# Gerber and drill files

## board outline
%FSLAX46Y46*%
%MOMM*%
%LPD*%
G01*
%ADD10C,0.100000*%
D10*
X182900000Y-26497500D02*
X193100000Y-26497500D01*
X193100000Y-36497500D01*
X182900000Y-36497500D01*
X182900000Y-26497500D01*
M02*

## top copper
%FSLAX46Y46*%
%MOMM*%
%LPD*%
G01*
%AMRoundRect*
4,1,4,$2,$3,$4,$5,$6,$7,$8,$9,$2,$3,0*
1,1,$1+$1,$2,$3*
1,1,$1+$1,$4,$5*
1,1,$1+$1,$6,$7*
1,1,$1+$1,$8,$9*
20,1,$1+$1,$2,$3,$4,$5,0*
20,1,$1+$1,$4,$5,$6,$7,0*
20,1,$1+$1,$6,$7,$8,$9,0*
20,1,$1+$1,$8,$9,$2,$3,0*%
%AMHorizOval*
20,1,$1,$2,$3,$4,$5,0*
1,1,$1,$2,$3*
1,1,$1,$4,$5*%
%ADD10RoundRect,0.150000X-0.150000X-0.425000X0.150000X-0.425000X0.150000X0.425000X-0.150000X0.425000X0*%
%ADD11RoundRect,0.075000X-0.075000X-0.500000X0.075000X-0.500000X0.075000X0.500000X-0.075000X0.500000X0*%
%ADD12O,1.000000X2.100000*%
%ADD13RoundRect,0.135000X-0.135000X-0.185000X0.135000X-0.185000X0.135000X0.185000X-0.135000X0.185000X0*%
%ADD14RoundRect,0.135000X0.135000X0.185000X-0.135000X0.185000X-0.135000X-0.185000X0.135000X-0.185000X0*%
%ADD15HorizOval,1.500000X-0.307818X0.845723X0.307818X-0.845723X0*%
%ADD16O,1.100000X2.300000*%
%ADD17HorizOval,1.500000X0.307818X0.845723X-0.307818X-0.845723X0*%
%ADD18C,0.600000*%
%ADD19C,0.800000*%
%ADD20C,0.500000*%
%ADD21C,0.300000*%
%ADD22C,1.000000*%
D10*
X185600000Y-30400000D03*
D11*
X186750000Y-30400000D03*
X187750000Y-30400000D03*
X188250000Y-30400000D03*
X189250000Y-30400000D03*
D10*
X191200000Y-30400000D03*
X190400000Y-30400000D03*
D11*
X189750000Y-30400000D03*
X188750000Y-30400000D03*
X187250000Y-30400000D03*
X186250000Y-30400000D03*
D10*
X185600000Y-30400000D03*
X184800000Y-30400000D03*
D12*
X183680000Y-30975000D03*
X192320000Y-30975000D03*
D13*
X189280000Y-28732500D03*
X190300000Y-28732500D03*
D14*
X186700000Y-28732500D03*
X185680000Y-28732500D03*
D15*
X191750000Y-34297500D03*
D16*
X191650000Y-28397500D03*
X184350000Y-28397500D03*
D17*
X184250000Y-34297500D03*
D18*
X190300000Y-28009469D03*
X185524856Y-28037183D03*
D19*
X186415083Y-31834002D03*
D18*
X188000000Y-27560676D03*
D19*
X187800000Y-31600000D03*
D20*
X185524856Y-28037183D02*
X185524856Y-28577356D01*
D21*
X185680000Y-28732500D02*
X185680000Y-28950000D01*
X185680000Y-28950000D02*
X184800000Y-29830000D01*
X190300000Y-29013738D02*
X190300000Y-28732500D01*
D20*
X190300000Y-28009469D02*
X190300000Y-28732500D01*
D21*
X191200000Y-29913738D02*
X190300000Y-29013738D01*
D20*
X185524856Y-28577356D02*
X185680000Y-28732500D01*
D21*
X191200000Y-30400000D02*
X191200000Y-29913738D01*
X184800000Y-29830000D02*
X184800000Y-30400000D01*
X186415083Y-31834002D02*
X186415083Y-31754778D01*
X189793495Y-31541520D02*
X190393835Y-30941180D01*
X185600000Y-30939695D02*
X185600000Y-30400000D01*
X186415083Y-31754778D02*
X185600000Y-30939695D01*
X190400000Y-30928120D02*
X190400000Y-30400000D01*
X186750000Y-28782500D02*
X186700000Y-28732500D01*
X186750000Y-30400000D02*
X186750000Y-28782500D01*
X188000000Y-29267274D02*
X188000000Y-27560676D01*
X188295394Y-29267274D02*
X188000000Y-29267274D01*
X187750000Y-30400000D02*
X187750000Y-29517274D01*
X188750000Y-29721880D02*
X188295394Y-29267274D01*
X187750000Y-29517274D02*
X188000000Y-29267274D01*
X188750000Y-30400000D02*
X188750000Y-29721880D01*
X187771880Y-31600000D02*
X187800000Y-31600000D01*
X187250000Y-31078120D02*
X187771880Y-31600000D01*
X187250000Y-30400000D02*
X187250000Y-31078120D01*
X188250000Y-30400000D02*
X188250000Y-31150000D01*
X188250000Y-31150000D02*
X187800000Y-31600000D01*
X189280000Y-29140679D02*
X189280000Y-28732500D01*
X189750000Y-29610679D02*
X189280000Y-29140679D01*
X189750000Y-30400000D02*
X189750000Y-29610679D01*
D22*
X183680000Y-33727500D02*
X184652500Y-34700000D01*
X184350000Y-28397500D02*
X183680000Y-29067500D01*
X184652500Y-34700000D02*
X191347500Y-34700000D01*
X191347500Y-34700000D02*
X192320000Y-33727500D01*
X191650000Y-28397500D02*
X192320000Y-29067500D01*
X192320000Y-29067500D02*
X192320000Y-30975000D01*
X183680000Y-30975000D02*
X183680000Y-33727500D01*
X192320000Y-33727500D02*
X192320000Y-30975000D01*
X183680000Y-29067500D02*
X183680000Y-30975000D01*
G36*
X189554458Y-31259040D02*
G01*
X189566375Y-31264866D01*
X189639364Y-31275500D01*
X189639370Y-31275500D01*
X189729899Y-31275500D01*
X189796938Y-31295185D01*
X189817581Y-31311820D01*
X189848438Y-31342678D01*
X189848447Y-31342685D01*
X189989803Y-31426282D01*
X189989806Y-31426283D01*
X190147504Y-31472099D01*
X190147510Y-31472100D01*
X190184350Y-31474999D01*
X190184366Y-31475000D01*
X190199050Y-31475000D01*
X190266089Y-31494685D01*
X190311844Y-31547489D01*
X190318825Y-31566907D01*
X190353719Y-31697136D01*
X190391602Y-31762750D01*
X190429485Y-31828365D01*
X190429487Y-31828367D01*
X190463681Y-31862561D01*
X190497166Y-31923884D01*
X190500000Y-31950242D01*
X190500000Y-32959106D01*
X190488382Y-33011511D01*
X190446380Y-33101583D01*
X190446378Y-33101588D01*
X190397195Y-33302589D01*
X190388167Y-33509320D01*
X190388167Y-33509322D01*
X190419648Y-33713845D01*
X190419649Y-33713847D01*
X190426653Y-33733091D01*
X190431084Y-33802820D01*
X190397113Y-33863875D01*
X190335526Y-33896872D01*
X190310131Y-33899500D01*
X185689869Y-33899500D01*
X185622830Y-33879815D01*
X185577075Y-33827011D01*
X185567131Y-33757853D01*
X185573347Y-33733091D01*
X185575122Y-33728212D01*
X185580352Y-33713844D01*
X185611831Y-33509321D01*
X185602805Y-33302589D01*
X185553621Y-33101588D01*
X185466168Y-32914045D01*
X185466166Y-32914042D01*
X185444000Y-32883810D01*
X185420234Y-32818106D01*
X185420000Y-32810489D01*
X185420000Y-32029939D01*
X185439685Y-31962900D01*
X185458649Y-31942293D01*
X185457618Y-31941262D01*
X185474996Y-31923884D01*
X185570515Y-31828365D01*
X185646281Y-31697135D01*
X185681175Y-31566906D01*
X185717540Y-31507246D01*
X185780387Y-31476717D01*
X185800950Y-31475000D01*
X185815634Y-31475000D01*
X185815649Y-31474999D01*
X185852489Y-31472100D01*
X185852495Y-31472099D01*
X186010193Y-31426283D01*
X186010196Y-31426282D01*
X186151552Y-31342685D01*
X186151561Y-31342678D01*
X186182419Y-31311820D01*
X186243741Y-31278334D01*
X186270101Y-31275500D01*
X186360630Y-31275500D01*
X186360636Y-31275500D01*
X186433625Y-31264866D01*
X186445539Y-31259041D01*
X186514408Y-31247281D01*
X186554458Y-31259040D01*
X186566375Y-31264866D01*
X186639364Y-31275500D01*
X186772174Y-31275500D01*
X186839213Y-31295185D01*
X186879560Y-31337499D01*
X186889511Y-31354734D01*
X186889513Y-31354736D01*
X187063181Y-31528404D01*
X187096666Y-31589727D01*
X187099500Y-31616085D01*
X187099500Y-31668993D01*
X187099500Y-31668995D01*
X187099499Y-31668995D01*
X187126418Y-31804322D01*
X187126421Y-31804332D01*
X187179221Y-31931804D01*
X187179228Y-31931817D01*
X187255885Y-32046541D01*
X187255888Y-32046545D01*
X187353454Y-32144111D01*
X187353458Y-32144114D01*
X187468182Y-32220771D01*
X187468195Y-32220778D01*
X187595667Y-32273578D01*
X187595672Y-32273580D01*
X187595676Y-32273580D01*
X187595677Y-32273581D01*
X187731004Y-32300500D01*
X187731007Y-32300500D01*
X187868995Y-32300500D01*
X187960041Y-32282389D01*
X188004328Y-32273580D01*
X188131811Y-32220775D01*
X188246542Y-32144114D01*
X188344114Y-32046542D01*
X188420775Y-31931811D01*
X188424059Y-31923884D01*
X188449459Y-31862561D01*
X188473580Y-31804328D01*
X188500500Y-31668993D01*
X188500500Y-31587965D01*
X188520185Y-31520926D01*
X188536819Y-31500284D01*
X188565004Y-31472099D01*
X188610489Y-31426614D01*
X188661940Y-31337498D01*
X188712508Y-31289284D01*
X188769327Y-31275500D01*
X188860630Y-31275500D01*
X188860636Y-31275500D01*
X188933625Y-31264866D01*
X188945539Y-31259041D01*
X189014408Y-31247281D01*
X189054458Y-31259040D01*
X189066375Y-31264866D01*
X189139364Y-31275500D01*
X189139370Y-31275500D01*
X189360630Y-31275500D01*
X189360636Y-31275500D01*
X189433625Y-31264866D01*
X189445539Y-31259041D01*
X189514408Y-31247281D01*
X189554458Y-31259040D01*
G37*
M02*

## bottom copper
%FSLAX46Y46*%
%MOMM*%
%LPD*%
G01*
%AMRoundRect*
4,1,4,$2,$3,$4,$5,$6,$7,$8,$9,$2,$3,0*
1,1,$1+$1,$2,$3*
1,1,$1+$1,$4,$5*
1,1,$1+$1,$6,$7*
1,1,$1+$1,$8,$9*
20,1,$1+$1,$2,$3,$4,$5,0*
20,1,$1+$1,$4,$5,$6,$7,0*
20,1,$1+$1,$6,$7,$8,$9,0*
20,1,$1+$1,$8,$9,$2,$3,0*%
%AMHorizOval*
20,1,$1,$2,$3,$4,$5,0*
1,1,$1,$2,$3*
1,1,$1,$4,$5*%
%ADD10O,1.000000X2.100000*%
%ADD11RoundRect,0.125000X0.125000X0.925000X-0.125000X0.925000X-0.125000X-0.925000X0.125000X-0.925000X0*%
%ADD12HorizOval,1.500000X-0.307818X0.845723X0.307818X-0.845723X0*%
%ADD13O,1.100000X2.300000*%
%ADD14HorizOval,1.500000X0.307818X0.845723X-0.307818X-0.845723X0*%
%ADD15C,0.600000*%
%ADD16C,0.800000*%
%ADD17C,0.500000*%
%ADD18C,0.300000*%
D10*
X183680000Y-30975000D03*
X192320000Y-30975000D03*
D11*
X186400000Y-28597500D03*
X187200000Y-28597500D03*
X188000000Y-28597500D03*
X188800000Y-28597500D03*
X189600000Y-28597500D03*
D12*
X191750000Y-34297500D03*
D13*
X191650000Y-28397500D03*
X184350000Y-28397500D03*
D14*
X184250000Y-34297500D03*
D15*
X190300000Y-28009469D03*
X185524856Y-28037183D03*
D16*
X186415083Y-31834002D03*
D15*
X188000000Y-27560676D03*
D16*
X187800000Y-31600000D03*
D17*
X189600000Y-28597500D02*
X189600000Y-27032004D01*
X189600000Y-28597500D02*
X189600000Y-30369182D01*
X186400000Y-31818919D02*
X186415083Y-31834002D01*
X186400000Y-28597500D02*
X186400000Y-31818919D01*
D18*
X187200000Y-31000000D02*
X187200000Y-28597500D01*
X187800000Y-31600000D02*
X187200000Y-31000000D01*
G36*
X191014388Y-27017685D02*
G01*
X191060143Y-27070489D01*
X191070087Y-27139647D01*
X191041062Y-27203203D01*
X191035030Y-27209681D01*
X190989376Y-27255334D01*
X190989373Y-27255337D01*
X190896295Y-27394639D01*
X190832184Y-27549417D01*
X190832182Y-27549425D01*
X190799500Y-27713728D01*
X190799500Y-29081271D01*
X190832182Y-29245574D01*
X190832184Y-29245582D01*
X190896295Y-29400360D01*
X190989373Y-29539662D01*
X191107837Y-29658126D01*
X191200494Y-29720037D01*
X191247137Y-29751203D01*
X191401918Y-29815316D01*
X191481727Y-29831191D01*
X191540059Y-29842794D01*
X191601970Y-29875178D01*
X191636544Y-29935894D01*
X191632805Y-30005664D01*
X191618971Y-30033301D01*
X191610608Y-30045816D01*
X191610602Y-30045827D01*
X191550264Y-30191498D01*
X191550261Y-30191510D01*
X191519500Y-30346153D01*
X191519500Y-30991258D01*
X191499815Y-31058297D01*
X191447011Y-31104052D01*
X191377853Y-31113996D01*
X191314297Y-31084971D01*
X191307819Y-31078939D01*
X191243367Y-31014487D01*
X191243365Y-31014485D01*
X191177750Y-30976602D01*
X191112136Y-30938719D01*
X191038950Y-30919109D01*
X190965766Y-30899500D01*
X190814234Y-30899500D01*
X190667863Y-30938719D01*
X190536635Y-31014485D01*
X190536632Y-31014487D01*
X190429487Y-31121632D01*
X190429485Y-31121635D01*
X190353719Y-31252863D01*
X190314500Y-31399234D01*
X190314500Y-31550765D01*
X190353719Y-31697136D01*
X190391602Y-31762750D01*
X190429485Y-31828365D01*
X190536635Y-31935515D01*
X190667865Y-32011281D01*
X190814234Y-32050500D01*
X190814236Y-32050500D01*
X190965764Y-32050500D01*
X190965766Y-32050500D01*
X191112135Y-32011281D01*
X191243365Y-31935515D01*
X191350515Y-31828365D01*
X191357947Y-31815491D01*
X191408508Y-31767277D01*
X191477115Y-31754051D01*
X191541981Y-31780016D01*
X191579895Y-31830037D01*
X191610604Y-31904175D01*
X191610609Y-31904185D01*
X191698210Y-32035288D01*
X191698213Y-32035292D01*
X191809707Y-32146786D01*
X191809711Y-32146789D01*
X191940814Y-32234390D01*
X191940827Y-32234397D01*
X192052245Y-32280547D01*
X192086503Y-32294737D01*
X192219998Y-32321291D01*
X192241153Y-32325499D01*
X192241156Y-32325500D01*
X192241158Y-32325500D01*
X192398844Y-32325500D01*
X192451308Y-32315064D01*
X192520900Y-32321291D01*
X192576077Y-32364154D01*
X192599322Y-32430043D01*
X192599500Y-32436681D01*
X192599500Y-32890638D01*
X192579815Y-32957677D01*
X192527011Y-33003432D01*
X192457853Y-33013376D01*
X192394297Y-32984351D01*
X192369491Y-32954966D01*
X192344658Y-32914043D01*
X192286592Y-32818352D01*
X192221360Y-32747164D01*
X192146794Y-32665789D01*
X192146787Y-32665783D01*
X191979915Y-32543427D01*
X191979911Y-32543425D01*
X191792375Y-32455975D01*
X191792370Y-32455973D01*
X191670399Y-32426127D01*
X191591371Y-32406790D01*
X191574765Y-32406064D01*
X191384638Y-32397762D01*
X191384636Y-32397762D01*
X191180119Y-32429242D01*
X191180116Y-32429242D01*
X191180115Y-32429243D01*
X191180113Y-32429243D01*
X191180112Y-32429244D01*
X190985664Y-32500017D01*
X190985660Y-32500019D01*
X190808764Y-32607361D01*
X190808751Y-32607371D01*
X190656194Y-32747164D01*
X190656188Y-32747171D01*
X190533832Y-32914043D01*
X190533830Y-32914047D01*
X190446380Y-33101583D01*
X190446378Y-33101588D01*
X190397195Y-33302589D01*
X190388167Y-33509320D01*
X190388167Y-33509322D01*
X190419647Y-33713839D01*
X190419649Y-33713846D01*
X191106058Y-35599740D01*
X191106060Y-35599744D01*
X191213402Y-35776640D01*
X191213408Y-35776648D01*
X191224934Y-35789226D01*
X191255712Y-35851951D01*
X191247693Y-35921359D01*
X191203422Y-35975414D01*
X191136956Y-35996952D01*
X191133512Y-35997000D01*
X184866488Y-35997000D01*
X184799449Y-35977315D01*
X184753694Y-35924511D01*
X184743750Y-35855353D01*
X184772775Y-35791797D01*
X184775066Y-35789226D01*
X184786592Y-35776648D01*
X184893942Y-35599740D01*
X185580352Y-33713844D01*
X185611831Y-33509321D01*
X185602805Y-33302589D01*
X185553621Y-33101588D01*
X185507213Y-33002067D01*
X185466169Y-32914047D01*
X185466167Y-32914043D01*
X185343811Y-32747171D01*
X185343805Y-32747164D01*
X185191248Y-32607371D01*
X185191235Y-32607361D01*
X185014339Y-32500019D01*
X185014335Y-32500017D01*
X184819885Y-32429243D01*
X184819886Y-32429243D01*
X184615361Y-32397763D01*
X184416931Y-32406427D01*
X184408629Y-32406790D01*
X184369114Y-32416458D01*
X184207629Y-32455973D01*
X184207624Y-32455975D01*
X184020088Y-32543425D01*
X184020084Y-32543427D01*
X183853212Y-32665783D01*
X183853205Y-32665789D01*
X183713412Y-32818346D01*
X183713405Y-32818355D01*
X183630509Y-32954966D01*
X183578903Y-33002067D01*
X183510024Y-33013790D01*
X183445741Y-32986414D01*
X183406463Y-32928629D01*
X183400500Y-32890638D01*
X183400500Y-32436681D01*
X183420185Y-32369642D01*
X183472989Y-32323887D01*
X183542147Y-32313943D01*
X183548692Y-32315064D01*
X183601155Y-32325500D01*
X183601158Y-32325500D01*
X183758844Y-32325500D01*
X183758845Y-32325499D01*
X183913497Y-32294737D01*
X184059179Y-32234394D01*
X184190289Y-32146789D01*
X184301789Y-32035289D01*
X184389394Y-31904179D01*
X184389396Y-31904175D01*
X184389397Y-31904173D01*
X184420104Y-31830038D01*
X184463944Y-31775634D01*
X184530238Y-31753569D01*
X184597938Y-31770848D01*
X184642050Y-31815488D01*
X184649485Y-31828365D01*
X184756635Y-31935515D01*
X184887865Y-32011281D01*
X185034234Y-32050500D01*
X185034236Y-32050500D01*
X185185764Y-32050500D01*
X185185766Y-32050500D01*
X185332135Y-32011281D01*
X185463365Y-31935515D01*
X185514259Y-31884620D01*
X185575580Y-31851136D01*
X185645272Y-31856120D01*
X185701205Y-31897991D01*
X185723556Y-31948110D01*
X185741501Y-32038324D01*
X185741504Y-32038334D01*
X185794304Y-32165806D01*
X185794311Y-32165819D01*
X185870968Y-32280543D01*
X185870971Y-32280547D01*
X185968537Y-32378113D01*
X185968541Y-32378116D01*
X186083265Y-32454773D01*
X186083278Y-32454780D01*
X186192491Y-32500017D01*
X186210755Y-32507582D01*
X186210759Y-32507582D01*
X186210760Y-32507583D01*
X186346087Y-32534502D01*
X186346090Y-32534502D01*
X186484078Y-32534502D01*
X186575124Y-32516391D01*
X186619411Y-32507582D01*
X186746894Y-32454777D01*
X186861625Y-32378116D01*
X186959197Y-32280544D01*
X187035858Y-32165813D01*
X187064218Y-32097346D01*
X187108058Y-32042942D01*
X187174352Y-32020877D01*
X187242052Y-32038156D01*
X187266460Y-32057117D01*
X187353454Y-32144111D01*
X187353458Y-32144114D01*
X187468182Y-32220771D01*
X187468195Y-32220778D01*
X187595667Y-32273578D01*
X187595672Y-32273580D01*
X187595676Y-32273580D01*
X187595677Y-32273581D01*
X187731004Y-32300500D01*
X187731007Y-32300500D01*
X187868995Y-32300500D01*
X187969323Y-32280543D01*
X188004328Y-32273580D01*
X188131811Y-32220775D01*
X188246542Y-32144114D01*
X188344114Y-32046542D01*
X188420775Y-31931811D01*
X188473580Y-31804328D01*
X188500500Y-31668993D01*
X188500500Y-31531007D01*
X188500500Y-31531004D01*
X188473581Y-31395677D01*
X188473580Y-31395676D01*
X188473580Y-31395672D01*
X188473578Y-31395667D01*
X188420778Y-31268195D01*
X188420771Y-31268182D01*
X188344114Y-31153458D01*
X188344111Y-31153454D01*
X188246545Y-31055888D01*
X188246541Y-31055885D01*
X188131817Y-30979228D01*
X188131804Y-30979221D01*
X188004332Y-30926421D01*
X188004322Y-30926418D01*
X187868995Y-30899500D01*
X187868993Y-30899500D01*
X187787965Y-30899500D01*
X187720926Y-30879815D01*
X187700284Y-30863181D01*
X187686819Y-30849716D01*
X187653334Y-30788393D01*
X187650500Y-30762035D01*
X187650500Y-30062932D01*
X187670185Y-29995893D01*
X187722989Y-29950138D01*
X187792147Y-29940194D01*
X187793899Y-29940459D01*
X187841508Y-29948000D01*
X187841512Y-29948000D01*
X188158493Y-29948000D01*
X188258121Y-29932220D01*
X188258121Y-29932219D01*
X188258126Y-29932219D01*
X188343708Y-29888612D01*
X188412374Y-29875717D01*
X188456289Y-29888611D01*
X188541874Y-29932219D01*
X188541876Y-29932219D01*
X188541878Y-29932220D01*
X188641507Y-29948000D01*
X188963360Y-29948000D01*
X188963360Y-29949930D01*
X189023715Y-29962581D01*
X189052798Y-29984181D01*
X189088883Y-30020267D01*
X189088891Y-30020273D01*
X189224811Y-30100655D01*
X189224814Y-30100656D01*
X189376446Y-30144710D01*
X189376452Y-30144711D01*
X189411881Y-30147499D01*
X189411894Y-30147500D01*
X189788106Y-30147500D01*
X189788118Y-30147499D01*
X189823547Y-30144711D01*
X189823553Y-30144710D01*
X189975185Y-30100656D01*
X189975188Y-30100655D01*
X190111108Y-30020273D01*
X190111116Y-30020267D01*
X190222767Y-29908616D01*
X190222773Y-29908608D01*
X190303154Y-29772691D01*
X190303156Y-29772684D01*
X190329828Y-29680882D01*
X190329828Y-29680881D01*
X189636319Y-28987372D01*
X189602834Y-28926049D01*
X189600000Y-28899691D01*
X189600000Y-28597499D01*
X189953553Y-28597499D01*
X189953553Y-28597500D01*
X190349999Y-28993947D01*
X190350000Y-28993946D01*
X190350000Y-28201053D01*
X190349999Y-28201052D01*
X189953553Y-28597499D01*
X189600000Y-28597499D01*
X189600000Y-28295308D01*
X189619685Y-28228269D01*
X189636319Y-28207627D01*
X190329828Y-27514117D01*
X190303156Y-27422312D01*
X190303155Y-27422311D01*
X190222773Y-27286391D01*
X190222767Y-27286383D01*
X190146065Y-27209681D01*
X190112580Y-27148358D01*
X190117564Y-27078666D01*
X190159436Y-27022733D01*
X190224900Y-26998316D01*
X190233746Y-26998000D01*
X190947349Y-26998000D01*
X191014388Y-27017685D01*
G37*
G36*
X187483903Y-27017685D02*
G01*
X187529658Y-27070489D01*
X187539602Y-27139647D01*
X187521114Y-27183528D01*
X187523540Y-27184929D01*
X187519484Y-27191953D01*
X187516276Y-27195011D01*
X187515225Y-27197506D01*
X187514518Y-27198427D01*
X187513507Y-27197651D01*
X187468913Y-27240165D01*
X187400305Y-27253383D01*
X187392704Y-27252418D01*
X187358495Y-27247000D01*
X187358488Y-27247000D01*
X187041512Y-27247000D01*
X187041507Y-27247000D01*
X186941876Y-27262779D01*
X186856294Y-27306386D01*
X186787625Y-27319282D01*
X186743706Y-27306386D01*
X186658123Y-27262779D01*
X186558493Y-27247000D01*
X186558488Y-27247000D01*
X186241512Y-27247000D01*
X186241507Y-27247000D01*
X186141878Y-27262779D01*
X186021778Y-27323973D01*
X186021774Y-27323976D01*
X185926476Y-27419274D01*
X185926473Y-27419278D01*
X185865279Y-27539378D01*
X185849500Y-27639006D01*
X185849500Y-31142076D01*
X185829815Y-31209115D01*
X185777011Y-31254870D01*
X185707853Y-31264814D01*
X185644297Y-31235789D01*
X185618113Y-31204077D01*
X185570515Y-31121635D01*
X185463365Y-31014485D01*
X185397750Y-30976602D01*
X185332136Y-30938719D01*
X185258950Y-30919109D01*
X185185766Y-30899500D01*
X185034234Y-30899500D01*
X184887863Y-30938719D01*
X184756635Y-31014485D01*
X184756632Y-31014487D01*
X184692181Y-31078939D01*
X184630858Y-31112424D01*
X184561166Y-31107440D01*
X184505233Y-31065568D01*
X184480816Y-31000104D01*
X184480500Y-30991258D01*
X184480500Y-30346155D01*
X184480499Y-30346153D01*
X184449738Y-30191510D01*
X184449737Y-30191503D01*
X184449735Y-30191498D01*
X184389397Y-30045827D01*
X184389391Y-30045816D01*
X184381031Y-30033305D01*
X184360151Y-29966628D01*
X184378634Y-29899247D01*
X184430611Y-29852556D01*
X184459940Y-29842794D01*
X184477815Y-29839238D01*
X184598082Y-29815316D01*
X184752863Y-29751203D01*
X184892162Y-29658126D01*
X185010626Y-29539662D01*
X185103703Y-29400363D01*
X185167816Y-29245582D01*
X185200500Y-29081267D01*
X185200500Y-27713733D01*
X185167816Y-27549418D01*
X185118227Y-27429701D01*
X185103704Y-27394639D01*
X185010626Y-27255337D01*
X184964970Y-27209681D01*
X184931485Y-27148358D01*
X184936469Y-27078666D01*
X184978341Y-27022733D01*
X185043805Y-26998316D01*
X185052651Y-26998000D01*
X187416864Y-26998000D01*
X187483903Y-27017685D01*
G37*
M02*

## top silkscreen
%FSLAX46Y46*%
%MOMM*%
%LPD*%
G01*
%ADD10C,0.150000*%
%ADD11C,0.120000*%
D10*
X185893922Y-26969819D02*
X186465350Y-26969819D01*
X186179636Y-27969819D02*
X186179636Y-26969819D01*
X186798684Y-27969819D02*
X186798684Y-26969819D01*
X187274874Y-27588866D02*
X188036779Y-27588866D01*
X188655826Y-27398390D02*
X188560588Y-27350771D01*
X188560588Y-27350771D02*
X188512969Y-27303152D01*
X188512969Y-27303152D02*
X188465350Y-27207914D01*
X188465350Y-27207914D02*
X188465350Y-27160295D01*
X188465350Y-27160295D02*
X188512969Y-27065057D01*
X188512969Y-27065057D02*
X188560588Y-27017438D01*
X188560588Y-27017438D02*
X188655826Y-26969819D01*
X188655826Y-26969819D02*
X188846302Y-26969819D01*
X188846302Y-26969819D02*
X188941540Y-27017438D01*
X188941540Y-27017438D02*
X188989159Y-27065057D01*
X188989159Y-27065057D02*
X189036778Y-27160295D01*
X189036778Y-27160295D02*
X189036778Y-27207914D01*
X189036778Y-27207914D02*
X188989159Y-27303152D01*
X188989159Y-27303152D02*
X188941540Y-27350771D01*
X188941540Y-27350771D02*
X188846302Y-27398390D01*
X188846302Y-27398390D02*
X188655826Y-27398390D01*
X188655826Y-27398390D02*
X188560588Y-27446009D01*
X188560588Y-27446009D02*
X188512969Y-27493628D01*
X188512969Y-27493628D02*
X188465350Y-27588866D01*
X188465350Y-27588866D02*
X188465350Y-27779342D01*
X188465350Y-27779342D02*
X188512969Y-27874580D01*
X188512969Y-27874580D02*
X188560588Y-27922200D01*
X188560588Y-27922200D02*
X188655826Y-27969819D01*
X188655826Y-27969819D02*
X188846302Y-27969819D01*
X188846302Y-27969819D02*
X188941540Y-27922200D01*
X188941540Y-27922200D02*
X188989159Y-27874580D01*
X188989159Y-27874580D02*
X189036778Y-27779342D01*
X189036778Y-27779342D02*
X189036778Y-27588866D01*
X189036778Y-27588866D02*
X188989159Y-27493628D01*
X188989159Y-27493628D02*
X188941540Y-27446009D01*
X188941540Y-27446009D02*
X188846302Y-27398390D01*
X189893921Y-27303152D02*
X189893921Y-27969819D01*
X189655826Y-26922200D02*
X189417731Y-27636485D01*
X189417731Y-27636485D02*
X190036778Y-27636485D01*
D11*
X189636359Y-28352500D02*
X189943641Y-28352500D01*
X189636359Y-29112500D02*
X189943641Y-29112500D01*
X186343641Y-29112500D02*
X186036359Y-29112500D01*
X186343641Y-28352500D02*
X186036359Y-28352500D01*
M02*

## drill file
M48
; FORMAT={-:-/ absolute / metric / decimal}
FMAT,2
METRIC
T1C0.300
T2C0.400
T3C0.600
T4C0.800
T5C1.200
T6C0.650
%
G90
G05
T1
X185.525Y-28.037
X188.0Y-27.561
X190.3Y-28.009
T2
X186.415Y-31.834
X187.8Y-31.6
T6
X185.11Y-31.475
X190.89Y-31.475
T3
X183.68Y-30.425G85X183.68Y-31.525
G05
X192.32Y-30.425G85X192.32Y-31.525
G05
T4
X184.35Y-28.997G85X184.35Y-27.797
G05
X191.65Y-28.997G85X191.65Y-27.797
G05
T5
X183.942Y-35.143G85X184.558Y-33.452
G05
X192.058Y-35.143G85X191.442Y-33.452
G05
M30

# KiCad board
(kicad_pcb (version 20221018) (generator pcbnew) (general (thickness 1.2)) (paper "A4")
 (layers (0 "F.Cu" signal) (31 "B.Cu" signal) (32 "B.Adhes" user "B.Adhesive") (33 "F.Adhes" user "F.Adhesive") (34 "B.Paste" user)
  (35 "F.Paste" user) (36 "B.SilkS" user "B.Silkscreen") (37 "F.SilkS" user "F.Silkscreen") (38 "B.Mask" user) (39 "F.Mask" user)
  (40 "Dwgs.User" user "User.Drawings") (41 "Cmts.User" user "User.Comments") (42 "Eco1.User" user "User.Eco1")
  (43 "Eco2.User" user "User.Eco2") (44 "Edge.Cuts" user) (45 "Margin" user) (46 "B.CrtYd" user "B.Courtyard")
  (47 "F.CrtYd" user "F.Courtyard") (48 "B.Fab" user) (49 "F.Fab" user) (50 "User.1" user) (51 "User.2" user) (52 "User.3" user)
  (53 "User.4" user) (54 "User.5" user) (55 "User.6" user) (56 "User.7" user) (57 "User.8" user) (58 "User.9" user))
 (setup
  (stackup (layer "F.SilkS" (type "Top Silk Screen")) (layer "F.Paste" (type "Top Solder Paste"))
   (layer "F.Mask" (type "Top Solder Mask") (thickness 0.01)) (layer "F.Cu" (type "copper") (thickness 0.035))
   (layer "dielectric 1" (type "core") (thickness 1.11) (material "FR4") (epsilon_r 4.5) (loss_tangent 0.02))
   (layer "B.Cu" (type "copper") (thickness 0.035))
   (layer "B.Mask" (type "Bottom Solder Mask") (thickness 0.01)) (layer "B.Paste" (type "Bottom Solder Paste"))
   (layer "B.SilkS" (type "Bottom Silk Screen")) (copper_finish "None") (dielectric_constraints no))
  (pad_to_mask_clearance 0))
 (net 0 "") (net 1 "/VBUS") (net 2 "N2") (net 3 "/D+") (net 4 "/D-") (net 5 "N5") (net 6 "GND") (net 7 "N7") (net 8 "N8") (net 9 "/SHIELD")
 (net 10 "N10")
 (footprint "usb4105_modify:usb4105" (layer "F.Cu") (at 187.98 39.92)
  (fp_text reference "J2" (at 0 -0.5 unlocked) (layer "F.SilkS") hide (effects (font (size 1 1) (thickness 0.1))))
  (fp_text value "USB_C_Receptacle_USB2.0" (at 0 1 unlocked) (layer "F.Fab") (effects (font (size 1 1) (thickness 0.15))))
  (pad "" np_thru_hole circle (at -2.87 -8.445) (size 0.65 0.65) (drill 0.65) (layers "F&B.Cu" "*.Mask"))
  (pad "" np_thru_hole circle (at 2.91 -8.445) (size 0.65 0.65) (drill 0.65) (layers "F&B.Cu" "*.Mask"))
  (pad "A4" smd roundrect (at -2.38 -9.52) (size 0.6 1.15) (layers "F.Cu" "F.Paste" "F.Mask") (roundrect_rratio 0.25) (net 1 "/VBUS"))
  (pad "A5" smd roundrect (at -1.23 -9.52) (size 0.3 1.15) (layers "F.Cu" "F.Paste" "F.Mask") (roundrect_rratio 0.25) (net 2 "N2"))
  (pad "A6" smd roundrect (at -0.23 -9.52) (size 0.3 1.15) (layers "F.Cu" "F.Paste" "F.Mask") (roundrect_rratio 0.25) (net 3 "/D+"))
  (pad "A7" smd roundrect (at 0.27 -9.52) (size 0.3 1.15) (layers "F.Cu" "F.Paste" "F.Mask") (roundrect_rratio 0.25) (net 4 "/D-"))
  (pad "A8" smd roundrect (at 1.27 -9.52) (size 0.3 1.15) (layers "F.Cu" "F.Paste" "F.Mask") (roundrect_rratio 0.25) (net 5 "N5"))
  (pad "A12" smd roundrect (at 3.22 -9.52) (size 0.6 1.15) (layers "F.Cu" "F.Paste" "F.Mask") (roundrect_rratio 0.25) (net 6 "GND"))
  (pad "B4" smd roundrect (at 2.42 -9.52) (size 0.6 1.15) (layers "F.Cu" "F.Paste" "F.Mask") (roundrect_rratio 0.25) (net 1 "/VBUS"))
  (pad "B5" smd roundrect (at 1.77 -9.52) (size 0.3 1.15) (layers "F.Cu" "F.Paste" "F.Mask") (roundrect_rratio 0.25) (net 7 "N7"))
  (pad "B6" smd roundrect (at 0.77 -9.52) (size 0.3 1.15) (layers "F.Cu" "F.Paste" "F.Mask") (roundrect_rratio 0.25) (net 3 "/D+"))
  (pad "B7" smd roundrect (at -0.73 -9.52) (size 0.3 1.15) (layers "F.Cu" "F.Paste" "F.Mask") (roundrect_rratio 0.25) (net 4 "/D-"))
  (pad "B8" smd roundrect (at -1.73 -9.52) (size 0.3 1.15) (layers "F.Cu" "F.Paste" "F.Mask") (roundrect_rratio 0.25) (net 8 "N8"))
  (pad "B9" smd roundrect (at -2.38 -9.52) (size 0.6 1.15) (layers "F.Cu" "F.Paste" "F.Mask") (roundrect_rratio 0.25) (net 1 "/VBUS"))
  (pad "B12" smd roundrect (at -3.18 -9.52) (size 0.6 1.15) (layers "F.Cu" "F.Paste" "F.Mask") (roundrect_rratio 0.25) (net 6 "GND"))
  (pad "S1" thru_hole oval (at -4.3 -8.945) (size 1 2.1) (drill oval 0.6 1.7) (layers "*.Cu" "*.Mask" "F.Paste") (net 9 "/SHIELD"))
  (pad "S1" thru_hole oval (at 4.34 -8.945) (size 1 2.1) (drill oval 0.6 1.7) (layers "*.Cu" "*.Mask" "F.Paste") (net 9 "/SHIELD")))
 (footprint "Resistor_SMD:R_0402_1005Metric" (layer "F.Cu") (at 189.79 28.7325)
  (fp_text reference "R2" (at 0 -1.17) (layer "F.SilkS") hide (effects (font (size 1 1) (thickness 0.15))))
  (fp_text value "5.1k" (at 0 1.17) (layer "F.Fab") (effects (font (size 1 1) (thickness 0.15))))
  (fp_line (start -0.153641 -0.38) (end 0.153641 -0.38) (stroke (width 0.12) (type solid)) (layer "F.SilkS"))
  (fp_line (start -0.153641 0.38) (end 0.153641 0.38) (stroke (width 0.12) (type solid)) (layer "F.SilkS"))
  (pad "1" smd roundrect (at -0.51 0) (size 0.54 0.64) (layers "F.Cu" "F.Paste" "F.Mask") (roundrect_rratio 0.25) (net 7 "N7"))
  (pad "2" smd roundrect (at 0.51 0) (size 0.54 0.64) (layers "F.Cu" "F.Paste" "F.Mask") (roundrect_rratio 0.25) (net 6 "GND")))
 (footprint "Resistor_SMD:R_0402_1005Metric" (layer "F.Cu") (at 186.19 28.7325 180)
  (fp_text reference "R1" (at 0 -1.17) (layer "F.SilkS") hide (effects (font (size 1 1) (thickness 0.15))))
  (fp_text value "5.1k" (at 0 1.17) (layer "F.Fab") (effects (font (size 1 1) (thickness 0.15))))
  (fp_line (start -0.153641 -0.38) (end 0.153641 -0.38) (stroke (width 0.12) (type solid)) (layer "F.SilkS"))
  (fp_line (start -0.153641 0.38) (end 0.153641 0.38) (stroke (width 0.12) (type solid)) (layer "F.SilkS"))
  (pad "1" smd roundrect (at -0.51 0 180) (size 0.54 0.64) (layers "F.Cu" "F.Paste" "F.Mask") (roundrect_rratio 0.25) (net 2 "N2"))
  (pad "2" smd roundrect (at 0.51 0 180) (size 0.54 0.64) (layers "F.Cu" "F.Paste" "F.Mask") (roundrect_rratio 0.25) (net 6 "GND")))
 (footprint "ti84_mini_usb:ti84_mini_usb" (layer "B.Cu") (at 188.25 38.1975 180)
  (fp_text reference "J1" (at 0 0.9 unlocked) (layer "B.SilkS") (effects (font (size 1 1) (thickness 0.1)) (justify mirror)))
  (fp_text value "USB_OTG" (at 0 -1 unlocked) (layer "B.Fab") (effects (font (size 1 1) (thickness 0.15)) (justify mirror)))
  (pad "1" smd roundrect (at 1.85 9.6 180) (size 0.5 2.1) (layers "B.Cu" "B.Paste" "B.Mask") (roundrect_rratio 0.25) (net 1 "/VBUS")
   (thermal_bridge_angle 45))
  (pad "2" smd roundrect (at 1.05 9.6 180) (size 0.5 2.1) (layers "B.Cu" "B.Paste" "B.Mask") (roundrect_rratio 0.25) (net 4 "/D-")
   (thermal_bridge_angle 45))
  (pad "3" smd roundrect (at 0.25 9.6 180) (size 0.5 2.1) (layers "B.Cu" "B.Paste" "B.Mask") (roundrect_rratio 0.25) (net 3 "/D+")
   (thermal_bridge_angle 45))
  (pad "4" smd roundrect (at -0.55 9.6 180) (size 0.5 2.1) (layers "B.Cu" "B.Paste" "B.Mask") (roundrect_rratio 0.25) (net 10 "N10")
   (thermal_bridge_angle 45))
  (pad "5" smd roundrect (at -1.35 9.6 180) (size 0.5 2.1) (layers "B.Cu" "B.Paste" "B.Mask") (roundrect_rratio 0.25) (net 6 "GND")
   (thermal_bridge_angle 45))
  (pad "6" thru_hole oval (at -3.5 3.9 200) (size 1.5 3.3) (drill oval 1.2 3) (layers "*.Cu" "*.Mask") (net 9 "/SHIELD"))
  (pad "6" thru_hole oval (at -3.4 9.8 180) (size 1.1 2.3) (drill oval 0.8 2) (layers "*.Cu" "*.Mask") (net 9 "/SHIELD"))
  (pad "6" thru_hole oval (at 3.9 9.8 180) (size 1.1 2.3) (drill oval 0.8 2) (layers "*.Cu" "*.Mask") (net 9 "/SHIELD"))
  (pad "6" thru_hole oval (at 4 3.9 160) (size 1.5 3.3) (drill oval 1.2 3) (layers "*.Cu" "*.Mask") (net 9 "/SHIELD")))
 (gr_rect (start 182.9 26.4975) (end 193.1 36.4975) (stroke (width 0.1) (type default)) (fill none) (layer "Edge.Cuts"))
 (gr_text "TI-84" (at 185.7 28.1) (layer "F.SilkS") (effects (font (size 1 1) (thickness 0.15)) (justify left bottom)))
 (segment (start 185.524856 28.037183) (end 185.524856 28.577356) (width 0.5) (layer "F.Cu") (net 6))
 (segment (start 185.68 28.7325) (end 185.68 28.95) (width 0.3) (layer "F.Cu") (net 6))
 (segment (start 185.68 28.95) (end 184.8 29.83) (width 0.3) (layer "F.Cu") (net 6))
 (segment (start 190.3 29.013738) (end 190.3 28.7325) (width 0.3) (layer "F.Cu") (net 6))
 (segment (start 190.3 28.009469) (end 190.3 28.7325) (width 0.5) (layer "F.Cu") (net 6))
 (segment (start 191.2 29.913738) (end 190.3 29.013738) (width 0.3) (layer "F.Cu") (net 6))
 (segment (start 185.524856 28.577356) (end 185.68 28.7325) (width 0.5) (layer "F.Cu") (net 6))
 (segment (start 191.2 30.4) (end 191.2 29.913738) (width 0.3) (layer "F.Cu") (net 6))
 (segment (start 184.8 29.83) (end 184.8 30.4) (width 0.3) (layer "F.Cu") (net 6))
 (via (at 190.3 28.009469) (size 0.6) (drill 0.3) (layers "F.Cu" "B.Cu") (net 6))
 (via (at 185.524856 28.037183) (size 0.6) (drill 0.3) (layers "F.Cu" "B.Cu") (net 6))
 (segment (start 189.6 28.5975) (end 189.6 27.032004) (width 0.5) (layer "B.Cu") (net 6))
 (segment (start 189.6 28.5975) (end 189.6 30.369182) (width 0.5) (layer "B.Cu") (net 6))
 (segment (start 186.415083 31.834002) (end 186.415083 31.754778) (width 0.3) (layer "F.Cu") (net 1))
 (segment (start 189.793495 31.54152) (end 190.393835 30.94118) (width 0.3) (layer "F.Cu") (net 1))
 (segment (start 185.6 30.939695) (end 185.6 30.4) (width 0.3) (layer "F.Cu") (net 1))
 (segment (start 186.415083 31.754778) (end 185.6 30.939695) (width 0.3) (layer "F.Cu") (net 1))
 (segment (start 190.4 30.92812) (end 190.4 30.4) (width 0.3) (layer "F.Cu") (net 1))
 (via (at 186.415083 31.834002) (size 0.8) (drill 0.4) (layers "F.Cu" "B.Cu") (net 1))
 (segment (start 186.4 31.818919) (end 186.415083 31.834002) (width 0.5) (layer "B.Cu") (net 1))
 (segment (start 186.4 28.5975) (end 186.4 31.818919) (width 0.5) (layer "B.Cu") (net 1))
 (segment (start 186.75 28.7825) (end 186.7 28.7325) (width 0.3) (layer "F.Cu") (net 2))
 (segment (start 186.75 30.4) (end 186.75 28.7825) (width 0.3) (layer "F.Cu") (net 2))
 (segment (start 188 29.267274) (end 188 27.560676) (width 0.3) (layer "F.Cu") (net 3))
 (segment (start 188.295394 29.267274) (end 188 29.267274) (width 0.3) (layer "F.Cu") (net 3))
 (segment (start 187.75 30.4) (end 187.75 29.517274) (width 0.3) (layer "F.Cu") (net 3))
 (segment (start 188.75 29.72188) (end 188.295394 29.267274) (width 0.3) (layer "F.Cu") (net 3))
 (segment (start 187.75 29.517274) (end 188 29.267274) (width 0.3) (layer "F.Cu") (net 3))
 (segment (start 188.75 30.4) (end 188.75 29.72188) (width 0.3) (layer "F.Cu") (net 3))
 (via (at 188 27.560676) (size 0.6) (drill 0.3) (layers "F.Cu" "B.Cu") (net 3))
 (segment (start 187.77188 31.6) (end 187.8 31.6) (width 0.3) (layer "F.Cu") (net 4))
 (segment (start 187.25 31.07812) (end 187.77188 31.6) (width 0.3) (layer "F.Cu") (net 4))
 (segment (start 187.25 30.4) (end 187.25 31.07812) (width 0.3) (layer "F.Cu") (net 4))
 (segment (start 188.25 30.4) (end 188.25 31.15) (width 0.3) (layer "F.Cu") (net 4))
 (segment (start 188.25 31.15) (end 187.8 31.6) (width 0.3) (layer "F.Cu") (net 4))
 (via (at 187.8 31.6) (size 0.8) (drill 0.4) (layers "F.Cu" "B.Cu") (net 4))
 (segment (start 187.2 31) (end 187.2 28.5975) (width 0.3) (layer "B.Cu") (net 4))
 (segment (start 187.8 31.6) (end 187.2 31) (width 0.3) (layer "B.Cu") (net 4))
 (segment (start 189.28 29.140679) (end 189.28 28.7325) (width 0.3) (layer "F.Cu") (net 7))
 (segment (start 189.75 29.610679) (end 189.28 29.140679) (width 0.3) (layer "F.Cu") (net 7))
 (segment (start 189.75 30.4) (end 189.75 29.610679) (width 0.3) (layer "F.Cu") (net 7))
 (segment (start 183.68 33.7275) (end 184.6525 34.7) (width 1) (layer "F.Cu") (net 9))
 (segment (start 184.35 28.3975) (end 183.68 29.0675) (width 1) (layer "F.Cu") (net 9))
 (segment (start 184.6525 34.7) (end 191.3475 34.7) (width 1) (layer "F.Cu") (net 9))
 (segment (start 191.3475 34.7) (end 192.32 33.7275) (width 1) (layer "F.Cu") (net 9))
 (segment (start 191.65 28.3975) (end 192.32 29.0675) (width 1) (layer "F.Cu") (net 9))
 (segment (start 192.32 29.0675) (end 192.32 30.975) (width 1) (layer "F.Cu") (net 9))
 (segment (start 183.68 30.975) (end 183.68 33.7275) (width 1) (layer "F.Cu") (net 9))
 (segment (start 192.32 33.7275) (end 192.32 30.975) (width 1) (layer "F.Cu") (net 9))
 (segment (start 183.68 29.0675) (end 183.68 30.975) (width 1) (layer "F.Cu") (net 9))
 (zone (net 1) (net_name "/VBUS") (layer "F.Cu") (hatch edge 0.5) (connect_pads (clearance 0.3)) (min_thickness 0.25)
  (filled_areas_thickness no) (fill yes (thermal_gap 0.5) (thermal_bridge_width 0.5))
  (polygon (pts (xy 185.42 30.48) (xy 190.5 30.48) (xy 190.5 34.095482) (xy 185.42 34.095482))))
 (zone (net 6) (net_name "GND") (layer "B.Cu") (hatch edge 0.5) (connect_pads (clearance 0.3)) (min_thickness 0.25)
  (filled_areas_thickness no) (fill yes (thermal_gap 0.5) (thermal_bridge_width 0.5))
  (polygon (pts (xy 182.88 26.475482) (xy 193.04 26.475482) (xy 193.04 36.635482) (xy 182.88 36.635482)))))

